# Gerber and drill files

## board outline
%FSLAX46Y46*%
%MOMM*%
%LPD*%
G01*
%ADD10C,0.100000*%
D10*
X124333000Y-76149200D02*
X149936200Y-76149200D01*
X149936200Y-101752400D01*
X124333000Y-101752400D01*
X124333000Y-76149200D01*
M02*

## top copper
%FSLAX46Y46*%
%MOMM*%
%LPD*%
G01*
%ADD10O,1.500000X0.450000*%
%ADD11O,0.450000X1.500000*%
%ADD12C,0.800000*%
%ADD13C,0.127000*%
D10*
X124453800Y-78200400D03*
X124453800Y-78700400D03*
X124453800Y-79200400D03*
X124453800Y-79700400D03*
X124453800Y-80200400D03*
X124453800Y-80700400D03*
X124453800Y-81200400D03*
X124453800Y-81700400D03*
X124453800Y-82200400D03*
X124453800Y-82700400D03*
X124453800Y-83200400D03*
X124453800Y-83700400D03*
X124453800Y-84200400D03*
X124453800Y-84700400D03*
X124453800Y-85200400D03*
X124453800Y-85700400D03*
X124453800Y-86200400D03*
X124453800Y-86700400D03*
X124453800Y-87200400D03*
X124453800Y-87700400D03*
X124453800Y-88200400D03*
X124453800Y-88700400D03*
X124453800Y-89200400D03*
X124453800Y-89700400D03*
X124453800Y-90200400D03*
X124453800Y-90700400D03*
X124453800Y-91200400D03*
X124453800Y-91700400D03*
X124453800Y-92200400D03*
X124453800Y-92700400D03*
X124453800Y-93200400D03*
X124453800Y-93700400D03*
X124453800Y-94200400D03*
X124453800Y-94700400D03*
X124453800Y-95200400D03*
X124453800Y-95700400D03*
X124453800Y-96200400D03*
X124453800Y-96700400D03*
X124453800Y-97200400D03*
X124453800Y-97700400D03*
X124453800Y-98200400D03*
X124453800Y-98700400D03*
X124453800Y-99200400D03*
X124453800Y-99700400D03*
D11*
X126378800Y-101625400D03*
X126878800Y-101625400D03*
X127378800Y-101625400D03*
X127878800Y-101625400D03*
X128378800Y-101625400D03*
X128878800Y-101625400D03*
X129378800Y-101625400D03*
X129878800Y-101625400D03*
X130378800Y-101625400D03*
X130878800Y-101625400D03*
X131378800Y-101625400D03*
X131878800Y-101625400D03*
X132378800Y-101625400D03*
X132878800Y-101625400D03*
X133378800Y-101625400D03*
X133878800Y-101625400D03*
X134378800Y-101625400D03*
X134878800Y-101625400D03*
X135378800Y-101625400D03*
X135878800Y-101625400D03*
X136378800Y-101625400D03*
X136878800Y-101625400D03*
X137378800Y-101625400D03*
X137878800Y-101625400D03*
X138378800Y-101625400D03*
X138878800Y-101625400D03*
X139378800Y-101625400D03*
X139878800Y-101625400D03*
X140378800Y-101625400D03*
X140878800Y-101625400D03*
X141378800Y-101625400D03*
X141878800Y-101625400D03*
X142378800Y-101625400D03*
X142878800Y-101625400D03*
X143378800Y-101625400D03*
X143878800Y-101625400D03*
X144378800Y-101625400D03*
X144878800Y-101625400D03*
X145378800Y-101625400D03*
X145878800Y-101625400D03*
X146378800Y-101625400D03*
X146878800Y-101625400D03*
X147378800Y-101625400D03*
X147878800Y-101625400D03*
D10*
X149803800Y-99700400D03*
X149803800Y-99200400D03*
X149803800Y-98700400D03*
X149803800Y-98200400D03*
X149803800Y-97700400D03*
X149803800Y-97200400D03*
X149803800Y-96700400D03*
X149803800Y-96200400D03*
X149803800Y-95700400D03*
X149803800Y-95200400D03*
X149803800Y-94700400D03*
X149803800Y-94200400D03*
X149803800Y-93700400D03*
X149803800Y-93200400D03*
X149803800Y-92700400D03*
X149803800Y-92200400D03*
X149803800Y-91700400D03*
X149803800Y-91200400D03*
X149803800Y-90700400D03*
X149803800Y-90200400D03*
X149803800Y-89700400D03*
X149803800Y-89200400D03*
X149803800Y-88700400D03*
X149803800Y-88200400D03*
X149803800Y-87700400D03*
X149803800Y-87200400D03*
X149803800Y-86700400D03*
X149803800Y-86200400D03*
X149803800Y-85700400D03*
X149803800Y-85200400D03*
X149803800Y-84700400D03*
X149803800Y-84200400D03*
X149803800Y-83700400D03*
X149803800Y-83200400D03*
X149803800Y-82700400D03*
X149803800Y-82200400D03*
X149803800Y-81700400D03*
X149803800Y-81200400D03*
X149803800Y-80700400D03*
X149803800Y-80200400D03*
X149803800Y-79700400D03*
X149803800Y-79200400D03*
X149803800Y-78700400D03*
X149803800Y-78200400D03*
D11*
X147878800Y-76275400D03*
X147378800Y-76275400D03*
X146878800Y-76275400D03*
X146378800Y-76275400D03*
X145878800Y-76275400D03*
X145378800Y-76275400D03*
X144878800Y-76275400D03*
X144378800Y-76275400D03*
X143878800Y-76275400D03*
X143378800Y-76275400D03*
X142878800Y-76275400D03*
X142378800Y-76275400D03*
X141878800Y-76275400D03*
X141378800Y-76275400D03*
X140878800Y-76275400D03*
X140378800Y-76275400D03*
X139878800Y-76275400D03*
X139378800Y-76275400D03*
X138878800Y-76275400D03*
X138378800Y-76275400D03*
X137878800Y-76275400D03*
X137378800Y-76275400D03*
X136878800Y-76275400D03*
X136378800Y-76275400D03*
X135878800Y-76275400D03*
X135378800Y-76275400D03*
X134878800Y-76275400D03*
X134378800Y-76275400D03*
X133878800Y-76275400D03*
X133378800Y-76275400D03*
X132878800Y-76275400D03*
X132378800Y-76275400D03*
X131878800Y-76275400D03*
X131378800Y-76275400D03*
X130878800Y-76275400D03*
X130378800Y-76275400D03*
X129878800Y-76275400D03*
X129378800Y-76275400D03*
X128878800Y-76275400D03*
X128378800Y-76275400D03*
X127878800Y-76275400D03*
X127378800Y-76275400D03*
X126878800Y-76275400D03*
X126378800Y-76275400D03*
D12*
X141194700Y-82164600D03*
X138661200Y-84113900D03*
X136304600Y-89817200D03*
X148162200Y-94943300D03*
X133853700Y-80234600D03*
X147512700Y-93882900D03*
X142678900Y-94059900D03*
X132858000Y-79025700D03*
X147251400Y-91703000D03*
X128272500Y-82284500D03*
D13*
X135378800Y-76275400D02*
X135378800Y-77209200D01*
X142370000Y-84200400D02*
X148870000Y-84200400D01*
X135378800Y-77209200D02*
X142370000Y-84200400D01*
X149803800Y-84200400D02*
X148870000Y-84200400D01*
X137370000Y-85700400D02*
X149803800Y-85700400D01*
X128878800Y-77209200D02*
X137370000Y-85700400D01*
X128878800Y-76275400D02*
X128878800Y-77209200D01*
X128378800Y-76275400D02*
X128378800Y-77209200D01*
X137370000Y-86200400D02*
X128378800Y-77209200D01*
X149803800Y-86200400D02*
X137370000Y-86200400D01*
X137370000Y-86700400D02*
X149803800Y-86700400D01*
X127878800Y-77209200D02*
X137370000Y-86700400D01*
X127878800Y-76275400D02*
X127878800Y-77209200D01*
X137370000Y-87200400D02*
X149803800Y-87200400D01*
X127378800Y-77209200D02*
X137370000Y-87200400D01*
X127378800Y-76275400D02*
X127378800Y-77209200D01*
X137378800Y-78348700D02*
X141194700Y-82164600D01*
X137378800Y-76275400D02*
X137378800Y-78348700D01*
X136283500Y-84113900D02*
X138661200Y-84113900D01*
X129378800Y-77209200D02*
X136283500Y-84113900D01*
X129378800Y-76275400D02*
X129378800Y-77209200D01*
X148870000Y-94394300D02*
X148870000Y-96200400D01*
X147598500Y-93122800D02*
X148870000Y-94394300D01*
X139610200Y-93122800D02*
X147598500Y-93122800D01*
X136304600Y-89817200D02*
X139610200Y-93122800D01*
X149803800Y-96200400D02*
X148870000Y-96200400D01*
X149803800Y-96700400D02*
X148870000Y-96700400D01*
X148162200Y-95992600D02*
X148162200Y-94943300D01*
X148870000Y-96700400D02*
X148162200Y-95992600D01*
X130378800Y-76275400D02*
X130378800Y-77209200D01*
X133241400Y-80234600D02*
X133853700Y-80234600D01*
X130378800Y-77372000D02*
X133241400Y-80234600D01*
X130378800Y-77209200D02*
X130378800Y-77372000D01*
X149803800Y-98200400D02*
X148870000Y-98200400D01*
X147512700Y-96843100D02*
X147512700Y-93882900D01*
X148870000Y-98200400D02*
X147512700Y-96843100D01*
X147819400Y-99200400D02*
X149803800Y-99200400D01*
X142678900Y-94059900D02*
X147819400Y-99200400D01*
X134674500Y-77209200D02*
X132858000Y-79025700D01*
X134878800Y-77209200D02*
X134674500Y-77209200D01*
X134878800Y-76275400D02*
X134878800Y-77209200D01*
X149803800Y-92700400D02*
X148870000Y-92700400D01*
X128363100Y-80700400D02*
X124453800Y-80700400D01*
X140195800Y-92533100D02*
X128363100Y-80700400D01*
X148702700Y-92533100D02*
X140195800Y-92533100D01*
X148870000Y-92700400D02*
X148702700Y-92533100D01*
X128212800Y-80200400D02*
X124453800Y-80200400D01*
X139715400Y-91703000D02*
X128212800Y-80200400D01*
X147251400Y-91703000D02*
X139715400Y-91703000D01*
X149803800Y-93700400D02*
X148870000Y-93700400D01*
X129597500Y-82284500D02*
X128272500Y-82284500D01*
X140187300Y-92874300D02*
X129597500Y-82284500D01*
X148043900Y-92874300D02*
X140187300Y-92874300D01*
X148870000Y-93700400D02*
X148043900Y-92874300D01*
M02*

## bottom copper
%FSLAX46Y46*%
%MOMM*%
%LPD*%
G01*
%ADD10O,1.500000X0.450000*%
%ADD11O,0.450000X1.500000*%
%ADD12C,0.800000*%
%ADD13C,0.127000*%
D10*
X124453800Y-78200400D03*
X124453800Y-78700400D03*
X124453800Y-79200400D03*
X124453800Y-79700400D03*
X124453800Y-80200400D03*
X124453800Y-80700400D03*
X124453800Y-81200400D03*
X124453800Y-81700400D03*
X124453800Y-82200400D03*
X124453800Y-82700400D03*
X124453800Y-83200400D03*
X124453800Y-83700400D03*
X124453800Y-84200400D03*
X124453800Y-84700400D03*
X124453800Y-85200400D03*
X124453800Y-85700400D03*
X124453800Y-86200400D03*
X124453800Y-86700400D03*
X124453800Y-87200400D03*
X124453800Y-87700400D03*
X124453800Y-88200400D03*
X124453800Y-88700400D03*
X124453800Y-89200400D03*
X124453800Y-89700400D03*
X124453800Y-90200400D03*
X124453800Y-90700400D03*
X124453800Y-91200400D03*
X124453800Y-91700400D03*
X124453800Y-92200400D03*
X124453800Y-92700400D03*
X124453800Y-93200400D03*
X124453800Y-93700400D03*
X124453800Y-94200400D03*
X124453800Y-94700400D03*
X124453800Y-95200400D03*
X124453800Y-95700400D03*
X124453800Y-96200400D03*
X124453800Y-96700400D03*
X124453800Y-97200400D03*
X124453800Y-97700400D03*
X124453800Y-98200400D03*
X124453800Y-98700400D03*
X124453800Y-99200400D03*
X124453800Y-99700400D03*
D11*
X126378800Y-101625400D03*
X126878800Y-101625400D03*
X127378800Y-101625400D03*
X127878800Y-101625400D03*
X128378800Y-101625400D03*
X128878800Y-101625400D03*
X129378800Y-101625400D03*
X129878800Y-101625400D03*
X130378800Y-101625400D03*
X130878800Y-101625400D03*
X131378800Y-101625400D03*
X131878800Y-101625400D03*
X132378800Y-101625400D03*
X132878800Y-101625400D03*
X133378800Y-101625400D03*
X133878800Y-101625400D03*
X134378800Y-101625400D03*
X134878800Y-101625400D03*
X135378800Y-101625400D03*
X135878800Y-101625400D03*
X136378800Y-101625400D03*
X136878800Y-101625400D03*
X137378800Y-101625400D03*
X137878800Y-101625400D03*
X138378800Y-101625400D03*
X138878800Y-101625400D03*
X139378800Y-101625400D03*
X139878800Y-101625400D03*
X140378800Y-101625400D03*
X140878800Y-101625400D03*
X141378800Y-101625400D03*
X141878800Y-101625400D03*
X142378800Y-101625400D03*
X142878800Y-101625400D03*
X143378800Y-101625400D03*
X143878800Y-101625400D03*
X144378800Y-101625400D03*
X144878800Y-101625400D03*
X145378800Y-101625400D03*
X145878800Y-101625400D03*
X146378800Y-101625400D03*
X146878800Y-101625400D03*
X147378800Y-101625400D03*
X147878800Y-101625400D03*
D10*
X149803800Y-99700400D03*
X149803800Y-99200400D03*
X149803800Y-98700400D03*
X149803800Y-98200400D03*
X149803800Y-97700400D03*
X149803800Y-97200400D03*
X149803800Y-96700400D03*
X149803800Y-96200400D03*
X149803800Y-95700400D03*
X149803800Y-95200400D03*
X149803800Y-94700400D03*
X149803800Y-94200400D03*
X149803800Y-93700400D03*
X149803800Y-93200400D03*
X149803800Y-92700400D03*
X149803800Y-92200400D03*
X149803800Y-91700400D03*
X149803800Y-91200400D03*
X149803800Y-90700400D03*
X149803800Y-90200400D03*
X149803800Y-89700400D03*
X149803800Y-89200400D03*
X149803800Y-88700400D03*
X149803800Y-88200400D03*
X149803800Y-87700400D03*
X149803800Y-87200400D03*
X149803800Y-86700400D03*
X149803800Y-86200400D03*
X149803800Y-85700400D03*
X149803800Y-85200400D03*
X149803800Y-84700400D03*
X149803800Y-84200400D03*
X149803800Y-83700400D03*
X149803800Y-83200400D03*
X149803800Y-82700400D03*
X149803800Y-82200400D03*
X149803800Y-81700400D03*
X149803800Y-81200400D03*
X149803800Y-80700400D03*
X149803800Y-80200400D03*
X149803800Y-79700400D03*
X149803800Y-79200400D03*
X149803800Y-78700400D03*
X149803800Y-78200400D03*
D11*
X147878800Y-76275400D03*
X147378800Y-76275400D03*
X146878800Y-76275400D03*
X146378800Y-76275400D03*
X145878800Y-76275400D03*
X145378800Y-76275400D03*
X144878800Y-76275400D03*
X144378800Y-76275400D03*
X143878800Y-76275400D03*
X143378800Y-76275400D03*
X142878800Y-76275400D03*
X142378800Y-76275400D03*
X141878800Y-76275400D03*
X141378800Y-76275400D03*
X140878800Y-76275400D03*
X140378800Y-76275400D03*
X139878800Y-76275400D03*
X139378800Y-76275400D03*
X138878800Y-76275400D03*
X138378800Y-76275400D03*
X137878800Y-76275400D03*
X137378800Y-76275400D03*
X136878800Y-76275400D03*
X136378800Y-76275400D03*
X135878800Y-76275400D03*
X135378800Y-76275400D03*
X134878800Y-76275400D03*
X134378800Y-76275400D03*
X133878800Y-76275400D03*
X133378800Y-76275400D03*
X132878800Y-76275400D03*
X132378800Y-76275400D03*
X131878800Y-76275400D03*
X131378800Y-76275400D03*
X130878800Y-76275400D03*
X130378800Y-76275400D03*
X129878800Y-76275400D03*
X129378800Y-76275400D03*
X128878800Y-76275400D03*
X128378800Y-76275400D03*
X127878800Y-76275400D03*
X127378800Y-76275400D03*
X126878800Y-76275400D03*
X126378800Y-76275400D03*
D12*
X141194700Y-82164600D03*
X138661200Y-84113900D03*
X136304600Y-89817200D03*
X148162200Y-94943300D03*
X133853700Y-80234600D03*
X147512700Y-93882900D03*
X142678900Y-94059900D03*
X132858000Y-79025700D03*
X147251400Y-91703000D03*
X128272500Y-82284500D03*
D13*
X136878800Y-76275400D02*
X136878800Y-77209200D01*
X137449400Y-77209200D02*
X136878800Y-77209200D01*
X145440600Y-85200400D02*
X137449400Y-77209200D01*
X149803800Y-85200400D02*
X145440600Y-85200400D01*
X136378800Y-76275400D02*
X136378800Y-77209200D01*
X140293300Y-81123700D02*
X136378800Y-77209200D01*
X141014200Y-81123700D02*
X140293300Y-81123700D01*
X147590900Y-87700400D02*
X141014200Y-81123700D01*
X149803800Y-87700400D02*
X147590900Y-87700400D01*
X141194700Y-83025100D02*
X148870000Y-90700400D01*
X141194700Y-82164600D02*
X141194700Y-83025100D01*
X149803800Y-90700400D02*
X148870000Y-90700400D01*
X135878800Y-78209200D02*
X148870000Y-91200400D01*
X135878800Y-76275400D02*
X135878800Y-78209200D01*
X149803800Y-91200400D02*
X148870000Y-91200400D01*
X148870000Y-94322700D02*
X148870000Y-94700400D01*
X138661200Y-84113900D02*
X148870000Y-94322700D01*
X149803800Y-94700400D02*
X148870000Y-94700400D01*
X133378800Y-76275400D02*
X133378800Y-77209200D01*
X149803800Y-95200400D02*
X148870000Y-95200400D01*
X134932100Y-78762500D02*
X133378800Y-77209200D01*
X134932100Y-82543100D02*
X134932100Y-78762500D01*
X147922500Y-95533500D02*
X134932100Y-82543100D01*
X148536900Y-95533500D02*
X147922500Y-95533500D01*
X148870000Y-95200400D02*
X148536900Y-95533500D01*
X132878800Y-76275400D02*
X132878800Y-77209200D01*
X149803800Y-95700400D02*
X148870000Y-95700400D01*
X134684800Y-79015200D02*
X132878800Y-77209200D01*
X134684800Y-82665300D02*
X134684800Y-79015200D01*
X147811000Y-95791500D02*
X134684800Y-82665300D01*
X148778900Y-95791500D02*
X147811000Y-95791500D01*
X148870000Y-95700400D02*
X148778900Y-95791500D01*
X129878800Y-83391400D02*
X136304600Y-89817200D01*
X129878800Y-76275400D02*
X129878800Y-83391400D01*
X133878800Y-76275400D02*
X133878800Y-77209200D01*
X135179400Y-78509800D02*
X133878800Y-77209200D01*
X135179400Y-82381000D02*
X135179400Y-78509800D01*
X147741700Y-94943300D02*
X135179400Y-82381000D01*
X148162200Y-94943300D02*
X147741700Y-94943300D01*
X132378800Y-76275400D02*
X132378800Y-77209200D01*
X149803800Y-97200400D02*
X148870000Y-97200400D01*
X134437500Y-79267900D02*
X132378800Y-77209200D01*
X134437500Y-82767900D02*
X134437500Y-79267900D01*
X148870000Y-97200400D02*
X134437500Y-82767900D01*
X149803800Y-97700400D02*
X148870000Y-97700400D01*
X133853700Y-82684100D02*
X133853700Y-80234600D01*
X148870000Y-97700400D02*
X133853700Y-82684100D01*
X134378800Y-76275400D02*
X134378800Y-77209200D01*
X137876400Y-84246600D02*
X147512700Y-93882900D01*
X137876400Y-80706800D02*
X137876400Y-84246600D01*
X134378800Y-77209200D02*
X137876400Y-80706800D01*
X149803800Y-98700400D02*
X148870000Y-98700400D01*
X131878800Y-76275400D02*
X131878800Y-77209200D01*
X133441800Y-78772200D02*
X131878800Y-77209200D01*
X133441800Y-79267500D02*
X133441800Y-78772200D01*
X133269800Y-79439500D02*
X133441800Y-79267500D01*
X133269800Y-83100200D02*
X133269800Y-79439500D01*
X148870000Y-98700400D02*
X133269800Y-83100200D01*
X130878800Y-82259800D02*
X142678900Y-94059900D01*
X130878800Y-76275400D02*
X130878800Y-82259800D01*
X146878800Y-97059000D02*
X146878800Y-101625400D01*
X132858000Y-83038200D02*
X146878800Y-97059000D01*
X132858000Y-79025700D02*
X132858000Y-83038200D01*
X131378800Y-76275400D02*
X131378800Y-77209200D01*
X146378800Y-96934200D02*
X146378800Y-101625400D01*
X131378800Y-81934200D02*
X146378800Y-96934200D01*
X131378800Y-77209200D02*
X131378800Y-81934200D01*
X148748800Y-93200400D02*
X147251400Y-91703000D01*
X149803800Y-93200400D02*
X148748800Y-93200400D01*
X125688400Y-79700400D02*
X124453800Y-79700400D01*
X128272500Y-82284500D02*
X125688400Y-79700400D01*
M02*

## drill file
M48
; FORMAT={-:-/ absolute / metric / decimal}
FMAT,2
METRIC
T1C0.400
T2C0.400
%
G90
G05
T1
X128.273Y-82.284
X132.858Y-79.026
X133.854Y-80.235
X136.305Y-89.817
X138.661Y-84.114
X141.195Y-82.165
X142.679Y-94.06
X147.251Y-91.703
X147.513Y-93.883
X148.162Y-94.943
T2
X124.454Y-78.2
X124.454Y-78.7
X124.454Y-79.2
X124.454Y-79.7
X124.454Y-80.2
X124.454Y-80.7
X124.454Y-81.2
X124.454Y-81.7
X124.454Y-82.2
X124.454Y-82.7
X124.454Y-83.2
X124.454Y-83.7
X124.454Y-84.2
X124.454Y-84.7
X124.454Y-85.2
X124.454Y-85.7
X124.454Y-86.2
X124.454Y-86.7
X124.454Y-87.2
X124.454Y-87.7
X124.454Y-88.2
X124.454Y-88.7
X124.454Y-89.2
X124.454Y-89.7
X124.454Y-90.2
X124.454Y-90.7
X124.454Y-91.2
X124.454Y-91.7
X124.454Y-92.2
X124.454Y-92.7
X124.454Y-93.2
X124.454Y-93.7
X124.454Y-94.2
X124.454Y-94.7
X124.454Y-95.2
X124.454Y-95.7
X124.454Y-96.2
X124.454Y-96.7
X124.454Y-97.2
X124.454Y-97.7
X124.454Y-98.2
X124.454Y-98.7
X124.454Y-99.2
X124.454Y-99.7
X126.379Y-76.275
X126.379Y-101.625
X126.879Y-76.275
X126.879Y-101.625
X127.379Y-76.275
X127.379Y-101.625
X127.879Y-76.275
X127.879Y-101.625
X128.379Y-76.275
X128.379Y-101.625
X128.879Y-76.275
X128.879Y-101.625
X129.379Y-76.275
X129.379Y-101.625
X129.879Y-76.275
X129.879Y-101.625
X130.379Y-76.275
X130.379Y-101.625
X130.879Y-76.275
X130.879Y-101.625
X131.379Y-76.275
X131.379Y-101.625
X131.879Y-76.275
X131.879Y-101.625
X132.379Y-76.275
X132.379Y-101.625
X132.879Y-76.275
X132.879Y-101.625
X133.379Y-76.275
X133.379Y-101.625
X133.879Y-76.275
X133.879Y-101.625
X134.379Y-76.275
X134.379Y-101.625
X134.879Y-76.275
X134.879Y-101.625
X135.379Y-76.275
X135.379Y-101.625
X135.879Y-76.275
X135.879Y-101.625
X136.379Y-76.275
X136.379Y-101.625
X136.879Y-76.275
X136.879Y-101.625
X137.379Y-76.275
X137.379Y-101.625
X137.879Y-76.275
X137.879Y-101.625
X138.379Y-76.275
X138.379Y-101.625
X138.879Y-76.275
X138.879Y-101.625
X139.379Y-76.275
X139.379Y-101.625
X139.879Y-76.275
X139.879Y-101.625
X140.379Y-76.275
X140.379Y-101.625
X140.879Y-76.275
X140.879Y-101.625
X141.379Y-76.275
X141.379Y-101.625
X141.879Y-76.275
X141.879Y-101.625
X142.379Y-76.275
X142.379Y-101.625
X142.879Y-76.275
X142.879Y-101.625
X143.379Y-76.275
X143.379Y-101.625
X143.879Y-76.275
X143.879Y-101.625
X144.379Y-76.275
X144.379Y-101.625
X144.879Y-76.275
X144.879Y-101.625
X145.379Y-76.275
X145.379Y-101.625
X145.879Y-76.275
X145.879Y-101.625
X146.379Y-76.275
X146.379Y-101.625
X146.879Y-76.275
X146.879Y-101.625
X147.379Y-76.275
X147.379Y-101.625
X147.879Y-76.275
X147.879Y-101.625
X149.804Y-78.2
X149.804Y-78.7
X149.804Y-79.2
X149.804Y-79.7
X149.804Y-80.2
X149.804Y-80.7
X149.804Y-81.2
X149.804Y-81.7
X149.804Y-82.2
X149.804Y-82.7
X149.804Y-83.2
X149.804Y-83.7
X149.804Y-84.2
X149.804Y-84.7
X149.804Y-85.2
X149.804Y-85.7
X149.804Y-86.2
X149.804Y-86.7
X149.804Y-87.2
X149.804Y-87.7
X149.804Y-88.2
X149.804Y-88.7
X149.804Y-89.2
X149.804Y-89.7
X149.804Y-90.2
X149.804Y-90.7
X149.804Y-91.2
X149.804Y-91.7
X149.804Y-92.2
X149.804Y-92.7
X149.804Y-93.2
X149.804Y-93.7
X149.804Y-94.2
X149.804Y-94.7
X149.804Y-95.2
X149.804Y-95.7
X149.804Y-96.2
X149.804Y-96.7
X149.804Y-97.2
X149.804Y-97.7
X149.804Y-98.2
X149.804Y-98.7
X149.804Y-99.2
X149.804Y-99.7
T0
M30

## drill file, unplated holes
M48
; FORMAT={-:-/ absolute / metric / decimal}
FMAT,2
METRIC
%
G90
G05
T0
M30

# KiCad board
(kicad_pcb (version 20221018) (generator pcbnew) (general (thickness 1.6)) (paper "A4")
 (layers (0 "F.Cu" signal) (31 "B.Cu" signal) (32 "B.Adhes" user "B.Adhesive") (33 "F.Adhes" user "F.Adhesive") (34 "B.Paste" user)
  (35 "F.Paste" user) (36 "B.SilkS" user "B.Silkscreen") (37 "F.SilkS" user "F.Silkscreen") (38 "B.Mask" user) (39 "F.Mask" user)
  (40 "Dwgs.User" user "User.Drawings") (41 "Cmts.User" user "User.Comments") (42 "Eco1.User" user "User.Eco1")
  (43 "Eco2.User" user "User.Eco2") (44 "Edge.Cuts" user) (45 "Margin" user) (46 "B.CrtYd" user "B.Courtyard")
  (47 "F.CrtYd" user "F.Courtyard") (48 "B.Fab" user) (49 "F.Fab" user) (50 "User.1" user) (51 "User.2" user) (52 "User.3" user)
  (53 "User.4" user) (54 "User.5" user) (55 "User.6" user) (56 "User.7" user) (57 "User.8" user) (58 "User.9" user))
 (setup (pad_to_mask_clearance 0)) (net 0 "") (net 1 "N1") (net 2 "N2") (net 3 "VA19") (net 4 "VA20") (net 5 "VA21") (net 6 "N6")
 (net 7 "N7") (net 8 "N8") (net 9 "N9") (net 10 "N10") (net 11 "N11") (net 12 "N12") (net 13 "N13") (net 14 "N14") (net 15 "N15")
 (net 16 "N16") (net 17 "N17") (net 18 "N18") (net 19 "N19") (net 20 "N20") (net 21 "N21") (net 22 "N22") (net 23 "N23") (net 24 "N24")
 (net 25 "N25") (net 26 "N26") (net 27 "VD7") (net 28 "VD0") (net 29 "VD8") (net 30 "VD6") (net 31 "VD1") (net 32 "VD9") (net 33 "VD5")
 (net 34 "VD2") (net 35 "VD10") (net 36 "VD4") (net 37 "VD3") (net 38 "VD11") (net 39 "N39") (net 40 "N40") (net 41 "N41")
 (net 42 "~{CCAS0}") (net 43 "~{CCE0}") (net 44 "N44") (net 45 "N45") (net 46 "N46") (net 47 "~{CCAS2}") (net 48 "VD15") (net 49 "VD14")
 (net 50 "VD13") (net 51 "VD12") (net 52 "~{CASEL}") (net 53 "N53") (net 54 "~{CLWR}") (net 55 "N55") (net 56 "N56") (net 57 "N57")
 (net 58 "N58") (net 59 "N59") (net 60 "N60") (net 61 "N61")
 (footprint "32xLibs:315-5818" (layer "F.Cu") (at 137.1288 88.9504)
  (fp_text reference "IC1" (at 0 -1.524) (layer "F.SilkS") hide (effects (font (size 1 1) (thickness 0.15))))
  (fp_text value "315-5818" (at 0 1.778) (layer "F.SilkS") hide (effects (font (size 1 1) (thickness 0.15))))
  (pad "1" thru_hole oval (at -12.675 -10.75) (size 1.5 0.45) (drill 0.4) (layers "*.Cu" "*.Mask"))
  (pad "2" thru_hole oval (at -12.675 -10.25) (size 1.5 0.45) (drill 0.4) (layers "*.Cu" "*.Mask") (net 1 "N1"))
  (pad "3" thru_hole oval (at -12.675 -9.75) (size 1.5 0.45) (drill 0.4) (layers "*.Cu" "*.Mask") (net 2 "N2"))
  (pad "4" thru_hole oval (at -12.675 -9.25) (size 1.5 0.45) (drill 0.4) (layers "*.Cu" "*.Mask") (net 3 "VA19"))
  (pad "5" thru_hole oval (at -12.675 -8.75) (size 1.5 0.45) (drill 0.4) (layers "*.Cu" "*.Mask") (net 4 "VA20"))
  (pad "6" thru_hole oval (at -12.675 -8.25) (size 1.5 0.45) (drill 0.4) (layers "*.Cu" "*.Mask") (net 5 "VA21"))
  (pad "7" thru_hole oval (at -12.675 -7.75) (size 1.5 0.45) (drill 0.4) (layers "*.Cu" "*.Mask") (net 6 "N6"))
  (pad "8" thru_hole oval (at -12.675 -7.25) (size 1.5 0.45) (drill 0.4) (layers "*.Cu" "*.Mask") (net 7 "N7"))
  (pad "9" thru_hole oval (at -12.675 -6.75) (size 1.5 0.45) (drill 0.4) (layers "*.Cu" "*.Mask"))
  (pad "10" thru_hole oval (at -12.675 -6.25) (size 1.5 0.45) (drill 0.4) (layers "*.Cu" "*.Mask"))
  (pad "11" thru_hole oval (at -12.675 -5.75) (size 1.5 0.45) (drill 0.4) (layers "*.Cu" "*.Mask"))
  (pad "12" thru_hole oval (at -12.675 -5.25) (size 1.5 0.45) (drill 0.4) (layers "*.Cu" "*.Mask"))
  (pad "13" thru_hole oval (at -12.675 -4.75) (size 1.5 0.45) (drill 0.4) (layers "*.Cu" "*.Mask"))
  (pad "14" thru_hole oval (at -12.675 -4.25) (size 1.5 0.45) (drill 0.4) (layers "*.Cu" "*.Mask"))
  (pad "15" thru_hole oval (at -12.675 -3.75) (size 1.5 0.45) (drill 0.4) (layers "*.Cu" "*.Mask"))
  (pad "16" thru_hole oval (at -12.675 -3.25) (size 1.5 0.45) (drill 0.4) (layers "*.Cu" "*.Mask"))
  (pad "17" thru_hole oval (at -12.675 -2.75) (size 1.5 0.45) (drill 0.4) (layers "*.Cu" "*.Mask"))
  (pad "18" thru_hole oval (at -12.675 -2.25) (size 1.5 0.45) (drill 0.4) (layers "*.Cu" "*.Mask"))
  (pad "19" thru_hole oval (at -12.675 -1.75) (size 1.5 0.45) (drill 0.4) (layers "*.Cu" "*.Mask"))
  (pad "20" thru_hole oval (at -12.675 -1.25) (size 1.5 0.45) (drill 0.4) (layers "*.Cu" "*.Mask"))
  (pad "21" thru_hole oval (at -12.675 -0.75) (size 1.5 0.45) (drill 0.4) (layers "*.Cu" "*.Mask"))
  (pad "22" thru_hole oval (at -12.675 -0.25) (size 1.5 0.45) (drill 0.4) (layers "*.Cu" "*.Mask"))
  (pad "23" thru_hole oval (at -12.675 0.25) (size 1.5 0.45) (drill 0.4) (layers "*.Cu" "*.Mask"))
  (pad "24" thru_hole oval (at -12.675 0.75) (size 1.5 0.45) (drill 0.4) (layers "*.Cu" "*.Mask"))
  (pad "25" thru_hole oval (at -12.675 1.25) (size 1.5 0.45) (drill 0.4) (layers "*.Cu" "*.Mask"))
  (pad "26" thru_hole oval (at -12.675 1.75) (size 1.5 0.45) (drill 0.4) (layers "*.Cu" "*.Mask"))
  (pad "27" thru_hole oval (at -12.675 2.25) (size 1.5 0.45) (drill 0.4) (layers "*.Cu" "*.Mask"))
  (pad "28" thru_hole oval (at -12.675 2.75) (size 1.5 0.45) (drill 0.4) (layers "*.Cu" "*.Mask"))
  (pad "29" thru_hole oval (at -12.675 3.25) (size 1.5 0.45) (drill 0.4) (layers "*.Cu" "*.Mask"))
  (pad "30" thru_hole oval (at -12.675 3.75) (size 1.5 0.45) (drill 0.4) (layers "*.Cu" "*.Mask"))
  (pad "31" thru_hole oval (at -12.675 4.25) (size 1.5 0.45) (drill 0.4) (layers "*.Cu" "*.Mask"))
  (pad "32" thru_hole oval (at -12.675 4.75) (size 1.5 0.45) (drill 0.4) (layers "*.Cu" "*.Mask"))
  (pad "33" thru_hole oval (at -12.675 5.25) (size 1.5 0.45) (drill 0.4) (layers "*.Cu" "*.Mask") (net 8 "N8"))
  (pad "34" thru_hole oval (at -12.675 5.75) (size 1.5 0.45) (drill 0.4) (layers "*.Cu" "*.Mask"))
  (pad "35" thru_hole oval (at -12.675 6.25) (size 1.5 0.45) (drill 0.4) (layers "*.Cu" "*.Mask"))
  (pad "36" thru_hole oval (at -12.675 6.75) (size 1.5 0.45) (drill 0.4) (layers "*.Cu" "*.Mask"))
  (pad "37" thru_hole oval (at -12.675 7.25) (size 1.5 0.45) (drill 0.4) (layers "*.Cu" "*.Mask"))
  (pad "38" thru_hole oval (at -12.675 7.75) (size 1.5 0.45) (drill 0.4) (layers "*.Cu" "*.Mask"))
  (pad "39" thru_hole oval (at -12.675 8.25) (size 1.5 0.45) (drill 0.4) (layers "*.Cu" "*.Mask"))
  (pad "40" thru_hole oval (at -12.675 8.75) (size 1.5 0.45) (drill 0.4) (layers "*.Cu" "*.Mask"))
  (pad "41" thru_hole oval (at -12.675 9.25) (size 1.5 0.45) (drill 0.4) (layers "*.Cu" "*.Mask"))
  (pad "42" thru_hole oval (at -12.675 9.75) (size 1.5 0.45) (drill 0.4) (layers "*.Cu" "*.Mask"))
  (pad "43" thru_hole oval (at -12.675 10.25) (size 1.5 0.45) (drill 0.4) (layers "*.Cu" "*.Mask"))
  (pad "44" thru_hole oval (at -12.675 10.75) (size 1.5 0.45) (drill 0.4) (layers "*.Cu" "*.Mask"))
  (pad "45" thru_hole oval (at -10.75 12.675) (size 0.45 1.5) (drill 0.4) (layers "*.Cu" "*.Mask"))
  (pad "46" thru_hole oval (at -10.25 12.675) (size 0.45 1.5) (drill 0.4) (layers "*.Cu" "*.Mask"))
  (pad "47" thru_hole oval (at -9.75 12.675) (size 0.45 1.5) (drill 0.4) (layers "*.Cu" "*.Mask"))
  (pad "48" thru_hole oval (at -9.25 12.675) (size 0.45 1.5) (drill 0.4) (layers "*.Cu" "*.Mask"))
  (pad "49" thru_hole oval (at -8.75 12.675) (size 0.45 1.5) (drill 0.4) (layers "*.Cu" "*.Mask"))
  (pad "50" thru_hole oval (at -8.25 12.675) (size 0.45 1.5) (drill 0.4) (layers "*.Cu" "*.Mask"))
  (pad "51" thru_hole oval (at -7.75 12.675) (size 0.45 1.5) (drill 0.4) (layers "*.Cu" "*.Mask"))
  (pad "52" thru_hole oval (at -7.25 12.675) (size 0.45 1.5) (drill 0.4) (layers "*.Cu" "*.Mask"))
  (pad "53" thru_hole oval (at -6.75 12.675) (size 0.45 1.5) (drill 0.4) (layers "*.Cu" "*.Mask"))
  (pad "54" thru_hole oval (at -6.25 12.675) (size 0.45 1.5) (drill 0.4) (layers "*.Cu" "*.Mask"))
  (pad "55" thru_hole oval (at -5.75 12.675) (size 0.45 1.5) (drill 0.4) (layers "*.Cu" "*.Mask"))
  (pad "56" thru_hole oval (at -5.25 12.675) (size 0.45 1.5) (drill 0.4) (layers "*.Cu" "*.Mask"))
  (pad "57" thru_hole oval (at -4.75 12.675) (size 0.45 1.5) (drill 0.4) (layers "*.Cu" "*.Mask"))
  (pad "58" thru_hole oval (at -4.25 12.675) (size 0.45 1.5) (drill 0.4) (layers "*.Cu" "*.Mask"))
  (pad "59" thru_hole oval (at -3.75 12.675) (size 0.45 1.5) (drill 0.4) (layers "*.Cu" "*.Mask"))
  (pad "60" thru_hole oval (at -3.25 12.675) (size 0.45 1.5) (drill 0.4) (layers "*.Cu" "*.Mask"))
  (pad "61" thru_hole oval (at -2.75 12.675) (size 0.45 1.5) (drill 0.4) (layers "*.Cu" "*.Mask"))
  (pad "62" thru_hole oval (at -2.25 12.675) (size 0.45 1.5) (drill 0.4) (layers "*.Cu" "*.Mask"))
  (pad "63" thru_hole oval (at -1.75 12.675) (size 0.45 1.5) (drill 0.4) (layers "*.Cu" "*.Mask"))
  (pad "64" thru_hole oval (at -1.25 12.675) (size 0.45 1.5) (drill 0.4) (layers "*.Cu" "*.Mask"))
  (pad "65" thru_hole oval (at -0.75 12.675) (size 0.45 1.5) (drill 0.4) (layers "*.Cu" "*.Mask"))
  (pad "66" thru_hole oval (at -0.25 12.675) (size 0.45 1.5) (drill 0.4) (layers "*.Cu" "*.Mask"))
  (pad "67" thru_hole oval (at 0.25 12.675) (size 0.45 1.5) (drill 0.4) (layers "*.Cu" "*.Mask") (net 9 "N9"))
  (pad "68" thru_hole oval (at 0.75 12.675) (size 0.45 1.5) (drill 0.4) (layers "*.Cu" "*.Mask") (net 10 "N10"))
  (pad "69" thru_hole oval (at 1.25 12.675) (size 0.45 1.5) (drill 0.4) (layers "*.Cu" "*.Mask") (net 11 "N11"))
  (pad "70" thru_hole oval (at 1.75 12.675) (size 0.45 1.5) (drill 0.4) (layers "*.Cu" "*.Mask") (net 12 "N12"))
  (pad "71" thru_hole oval (at 2.25 12.675) (size 0.45 1.5) (drill 0.4) (layers "*.Cu" "*.Mask") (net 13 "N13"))
  (pad "72" thru_hole oval (at 2.75 12.675) (size 0.45 1.5) (drill 0.4) (layers "*.Cu" "*.Mask") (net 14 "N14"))
  (pad "73" thru_hole oval (at 3.25 12.675) (size 0.45 1.5) (drill 0.4) (layers "*.Cu" "*.Mask") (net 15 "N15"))
  (pad "74" thru_hole oval (at 3.75 12.675) (size 0.45 1.5) (drill 0.4) (layers "*.Cu" "*.Mask") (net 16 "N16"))
  (pad "75" thru_hole oval (at 4.25 12.675) (size 0.45 1.5) (drill 0.4) (layers "*.Cu" "*.Mask") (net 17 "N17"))
  (pad "76" thru_hole oval (at 4.75 12.675) (size 0.45 1.5) (drill 0.4) (layers "*.Cu" "*.Mask") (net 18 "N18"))
  (pad "77" thru_hole oval (at 5.25 12.675) (size 0.45 1.5) (drill 0.4) (layers "*.Cu" "*.Mask") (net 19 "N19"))
  (pad "78" thru_hole oval (at 5.75 12.675) (size 0.45 1.5) (drill 0.4) (layers "*.Cu" "*.Mask") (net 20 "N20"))
  (pad "79" thru_hole oval (at 6.25 12.675) (size 0.45 1.5) (drill 0.4) (layers "*.Cu" "*.Mask") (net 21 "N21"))
  (pad "80" thru_hole oval (at 6.75 12.675) (size 0.45 1.5) (drill 0.4) (layers "*.Cu" "*.Mask") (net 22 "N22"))
  (pad "81" thru_hole oval (at 7.25 12.675) (size 0.45 1.5) (drill 0.4) (layers "*.Cu" "*.Mask") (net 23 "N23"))
  (pad "82" thru_hole oval (at 7.75 12.675) (size 0.45 1.5) (drill 0.4) (layers "*.Cu" "*.Mask") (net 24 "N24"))
  (pad "83" thru_hole oval (at 8.25 12.675) (size 0.45 1.5) (drill 0.4) (layers "*.Cu" "*.Mask") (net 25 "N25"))
  (pad "84" thru_hole oval (at 8.75 12.675) (size 0.45 1.5) (drill 0.4) (layers "*.Cu" "*.Mask") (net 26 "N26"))
  (pad "85" thru_hole oval (at 9.25 12.675) (size 0.45 1.5) (drill 0.4) (layers "*.Cu" "*.Mask") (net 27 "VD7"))
  (pad "86" thru_hole oval (at 9.75 12.675) (size 0.45 1.5) (drill 0.4) (layers "*.Cu" "*.Mask") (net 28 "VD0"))
  (pad "87" thru_hole oval (at 10.25 12.675) (size 0.45 1.5) (drill 0.4) (layers "*.Cu" "*.Mask"))
  (pad "88" thru_hole oval (at 10.75 12.675) (size 0.45 1.5) (drill 0.4) (layers "*.Cu" "*.Mask"))
  (pad "89" thru_hole oval (at 12.675 10.75) (size 1.5 0.45) (drill 0.4) (layers "*.Cu" "*.Mask"))
  (pad "90" thru_hole oval (at 12.675 10.25) (size 1.5 0.45) (drill 0.4) (layers "*.Cu" "*.Mask") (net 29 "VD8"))
  (pad "91" thru_hole oval (at 12.675 9.75) (size 1.5 0.45) (drill 0.4) (layers "*.Cu" "*.Mask") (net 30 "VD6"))
  (pad "92" thru_hole oval (at 12.675 9.25) (size 1.5 0.45) (drill 0.4) (layers "*.Cu" "*.Mask") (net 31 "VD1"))
  (pad "93" thru_hole oval (at 12.675 8.75) (size 1.5 0.45) (drill 0.4) (layers "*.Cu" "*.Mask") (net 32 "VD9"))
  (pad "94" thru_hole oval (at 12.675 8.25) (size 1.5 0.45) (drill 0.4) (layers "*.Cu" "*.Mask") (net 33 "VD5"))
  (pad "95" thru_hole oval (at 12.675 7.75) (size 1.5 0.45) (drill 0.4) (layers "*.Cu" "*.Mask") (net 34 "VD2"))
  (pad "96" thru_hole oval (at 12.675 7.25) (size 1.5 0.45) (drill 0.4) (layers "*.Cu" "*.Mask") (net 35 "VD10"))
  (pad "97" thru_hole oval (at 12.675 6.75) (size 1.5 0.45) (drill 0.4) (layers "*.Cu" "*.Mask") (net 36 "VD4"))
  (pad "98" thru_hole oval (at 12.675 6.25) (size 1.5 0.45) (drill 0.4) (layers "*.Cu" "*.Mask") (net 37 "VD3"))
  (pad "99" thru_hole oval (at 12.675 5.75) (size 1.5 0.45) (drill 0.4) (layers "*.Cu" "*.Mask") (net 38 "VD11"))
  (pad "100" thru_hole oval (at 12.675 5.25) (size 1.5 0.45) (drill 0.4) (layers "*.Cu" "*.Mask") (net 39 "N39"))
  (pad "101" thru_hole oval (at 12.675 4.75) (size 1.5 0.45) (drill 0.4) (layers "*.Cu" "*.Mask") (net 3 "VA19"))
  (pad "102" thru_hole oval (at 12.675 4.25) (size 1.5 0.45) (drill 0.4) (layers "*.Cu" "*.Mask") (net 4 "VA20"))
  (pad "103" thru_hole oval (at 12.675 3.75) (size 1.5 0.45) (drill 0.4) (layers "*.Cu" "*.Mask") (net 5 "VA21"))
  (pad "104" thru_hole oval (at 12.675 3.25) (size 1.5 0.45) (drill 0.4) (layers "*.Cu" "*.Mask") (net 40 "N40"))
  (pad "105" thru_hole oval (at 12.675 2.75) (size 1.5 0.45) (drill 0.4) (layers "*.Cu" "*.Mask") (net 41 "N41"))
  (pad "106" thru_hole oval (at 12.675 2.25) (size 1.5 0.45) (drill 0.4) (layers "*.Cu" "*.Mask") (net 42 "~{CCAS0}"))
  (pad "107" thru_hole oval (at 12.675 1.75) (size 1.5 0.45) (drill 0.4) (layers "*.Cu" "*.Mask") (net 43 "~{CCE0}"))
  (pad "108" thru_hole oval (at 12.675 1.25) (size 1.5 0.45) (drill 0.4) (layers "*.Cu" "*.Mask") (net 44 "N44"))
  (pad "109" thru_hole oval (at 12.675 0.75) (size 1.5 0.45) (drill 0.4) (layers "*.Cu" "*.Mask") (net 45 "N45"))
  (pad "110" thru_hole oval (at 12.675 0.25) (size 1.5 0.45) (drill 0.4) (layers "*.Cu" "*.Mask"))
  (pad "111" thru_hole oval (at 12.675 -0.25) (size 1.5 0.45) (drill 0.4) (layers "*.Cu" "*.Mask"))
  (pad "112" thru_hole oval (at 12.675 -0.75) (size 1.5 0.45) (drill 0.4) (layers "*.Cu" "*.Mask") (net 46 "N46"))
  (pad "113" thru_hole oval (at 12.675 -1.25) (size 1.5 0.45) (drill 0.4) (layers "*.Cu" "*.Mask") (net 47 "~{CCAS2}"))
  (pad "114" thru_hole oval (at 12.675 -1.75) (size 1.5 0.45) (drill 0.4) (layers "*.Cu" "*.Mask") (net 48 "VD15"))
  (pad "115" thru_hole oval (at 12.675 -2.25) (size 1.5 0.45) (drill 0.4) (layers "*.Cu" "*.Mask") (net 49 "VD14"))
  (pad "116" thru_hole oval (at 12.675 -2.75) (size 1.5 0.45) (drill 0.4) (layers "*.Cu" "*.Mask") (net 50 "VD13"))
  (pad "117" thru_hole oval (at 12.675 -3.25) (size 1.5 0.45) (drill 0.4) (layers "*.Cu" "*.Mask") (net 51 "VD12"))
  (pad "118" thru_hole oval (at 12.675 -3.75) (size 1.5 0.45) (drill 0.4) (layers "*.Cu" "*.Mask") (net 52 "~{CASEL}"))
  (pad "119" thru_hole oval (at 12.675 -4.25) (size 1.5 0.45) (drill 0.4) (layers "*.Cu" "*.Mask") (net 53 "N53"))
  (pad "120" thru_hole oval (at 12.675 -4.75) (size 1.5 0.45) (drill 0.4) (layers "*.Cu" "*.Mask") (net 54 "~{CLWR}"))
  (pad "121" thru_hole oval (at 12.675 -5.25) (size 1.5 0.45) (drill 0.4) (layers "*.Cu" "*.Mask") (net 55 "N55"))
  (pad "122" thru_hole oval (at 12.675 -5.75) (size 1.5 0.45) (drill 0.4) (layers "*.Cu" "*.Mask"))
  (pad "123" thru_hole oval (at 12.675 -6.25) (size 1.5 0.45) (drill 0.4) (layers "*.Cu" "*.Mask"))
  (pad "124" thru_hole oval (at 12.675 -6.75) (size 1.5 0.45) (drill 0.4) (layers "*.Cu" "*.Mask"))
  (pad "125" thru_hole oval (at 12.675 -7.25) (size 1.5 0.45) (drill 0.4) (layers "*.Cu" "*.Mask"))
  (pad "126" thru_hole oval (at 12.675 -7.75) (size 1.5 0.45) (drill 0.4) (layers "*.Cu" "*.Mask"))
  (pad "127" thru_hole oval (at 12.675 -8.25) (size 1.5 0.45) (drill 0.4) (layers "*.Cu" "*.Mask"))
  (pad "128" thru_hole oval (at 12.675 -8.75) (size 1.5 0.45) (drill 0.4) (layers "*.Cu" "*.Mask") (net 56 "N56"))
  (pad "129" thru_hole oval (at 12.675 -9.25) (size 1.5 0.45) (drill 0.4) (layers "*.Cu" "*.Mask") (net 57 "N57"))
  (pad "130" thru_hole oval (at 12.675 -9.75) (size 1.5 0.45) (drill 0.4) (layers "*.Cu" "*.Mask") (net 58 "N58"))
  (pad "131" thru_hole oval (at 12.675 -10.25) (size 1.5 0.45) (drill 0.4) (layers "*.Cu" "*.Mask"))
  (pad "132" thru_hole oval (at 12.675 -10.75) (size 1.5 0.45) (drill 0.4) (layers "*.Cu" "*.Mask"))
  (pad "133" thru_hole oval (at 10.75 -12.675) (size 0.45 1.5) (drill 0.4) (layers "*.Cu" "*.Mask"))
  (pad "134" thru_hole oval (at 10.25 -12.675) (size 0.45 1.5) (drill 0.4) (layers "*.Cu" "*.Mask"))
  (pad "135" thru_hole oval (at 9.75 -12.675) (size 0.45 1.5) (drill 0.4) (layers "*.Cu" "*.Mask"))
  (pad "136" thru_hole oval (at 9.25 -12.675) (size 0.45 1.5) (drill 0.4) (layers "*.Cu" "*.Mask"))
  (pad "137" thru_hole oval (at 8.75 -12.675) (size 0.45 1.5) (drill 0.4) (layers "*.Cu" "*.Mask"))
  (pad "138" thru_hole oval (at 8.25 -12.675) (size 0.45 1.5) (drill 0.4) (layers "*.Cu" "*.Mask"))
  (pad "139" thru_hole oval (at 7.75 -12.675) (size 0.45 1.5) (drill 0.4) (layers "*.Cu" "*.Mask"))
  (pad "140" thru_hole oval (at 7.25 -12.675) (size 0.45 1.5) (drill 0.4) (layers "*.Cu" "*.Mask"))
  (pad "141" thru_hole oval (at 6.75 -12.675) (size 0.45 1.5) (drill 0.4) (layers "*.Cu" "*.Mask"))
  (pad "142" thru_hole oval (at 6.25 -12.675) (size 0.45 1.5) (drill 0.4) (layers "*.Cu" "*.Mask"))
  (pad "143" thru_hole oval (at 5.75 -12.675) (size 0.45 1.5) (drill 0.4) (layers "*.Cu" "*.Mask"))
  (pad "144" thru_hole oval (at 5.25 -12.675) (size 0.45 1.5) (drill 0.4) (layers "*.Cu" "*.Mask"))
  (pad "145" thru_hole oval (at 4.75 -12.675) (size 0.45 1.5) (drill 0.4) (layers "*.Cu" "*.Mask"))
  (pad "146" thru_hole oval (at 4.25 -12.675) (size 0.45 1.5) (drill 0.4) (layers "*.Cu" "*.Mask"))
  (pad "147" thru_hole oval (at 3.75 -12.675) (size 0.45 1.5) (drill 0.4) (layers "*.Cu" "*.Mask"))
  (pad "148" thru_hole oval (at 3.25 -12.675) (size 0.45 1.5) (drill 0.4) (layers "*.Cu" "*.Mask"))
  (pad "149" thru_hole oval (at 2.75 -12.675) (size 0.45 1.5) (drill 0.4) (layers "*.Cu" "*.Mask"))
  (pad "150" thru_hole oval (at 2.25 -12.675) (size 0.45 1.5) (drill 0.4) (layers "*.Cu" "*.Mask"))
  (pad "151" thru_hole oval (at 1.75 -12.675) (size 0.45 1.5) (drill 0.4) (layers "*.Cu" "*.Mask") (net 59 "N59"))
  (pad "152" thru_hole oval (at 1.25 -12.675) (size 0.45 1.5) (drill 0.4) (layers "*.Cu" "*.Mask") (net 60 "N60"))
  (pad "153" thru_hole oval (at 0.75 -12.675) (size 0.45 1.5) (drill 0.4) (layers "*.Cu" "*.Mask") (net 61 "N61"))
  (pad "154" thru_hole oval (at 0.25 -12.675) (size 0.45 1.5) (drill 0.4) (layers "*.Cu" "*.Mask") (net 43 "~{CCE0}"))
  (pad "155" thru_hole oval (at -0.25 -12.675) (size 0.45 1.5) (drill 0.4) (layers "*.Cu" "*.Mask") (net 52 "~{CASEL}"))
  (pad "156" thru_hole oval (at -0.75 -12.675) (size 0.45 1.5) (drill 0.4) (layers "*.Cu" "*.Mask") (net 47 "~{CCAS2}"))
  (pad "157" thru_hole oval (at -1.25 -12.675) (size 0.45 1.5) (drill 0.4) (layers "*.Cu" "*.Mask") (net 42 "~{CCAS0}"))
  (pad "158" thru_hole oval (at -1.75 -12.675) (size 0.45 1.5) (drill 0.4) (layers "*.Cu" "*.Mask") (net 54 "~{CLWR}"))
  (pad "159" thru_hole oval (at -2.25 -12.675) (size 0.45 1.5) (drill 0.4) (layers "*.Cu" "*.Mask") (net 28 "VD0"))
  (pad "160" thru_hole oval (at -2.75 -12.675) (size 0.45 1.5) (drill 0.4) (layers "*.Cu" "*.Mask") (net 31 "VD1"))
  (pad "161" thru_hole oval (at -3.25 -12.675) (size 0.45 1.5) (drill 0.4) (layers "*.Cu" "*.Mask") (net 34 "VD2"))
  (pad "162" thru_hole oval (at -3.75 -12.675) (size 0.45 1.5) (drill 0.4) (layers "*.Cu" "*.Mask") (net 37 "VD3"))
  (pad "163" thru_hole oval (at -4.25 -12.675) (size 0.45 1.5) (drill 0.4) (layers "*.Cu" "*.Mask") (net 36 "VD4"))
  (pad "164" thru_hole oval (at -4.75 -12.675) (size 0.45 1.5) (drill 0.4) (layers "*.Cu" "*.Mask") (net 33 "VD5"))
  (pad "165" thru_hole oval (at -5.25 -12.675) (size 0.45 1.5) (drill 0.4) (layers "*.Cu" "*.Mask") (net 30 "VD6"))
  (pad "166" thru_hole oval (at -5.75 -12.675) (size 0.45 1.5) (drill 0.4) (layers "*.Cu" "*.Mask") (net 27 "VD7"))
  (pad "167" thru_hole oval (at -6.25 -12.675) (size 0.45 1.5) (drill 0.4) (layers "*.Cu" "*.Mask") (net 29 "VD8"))
  (pad "168" thru_hole oval (at -6.75 -12.675) (size 0.45 1.5) (drill 0.4) (layers "*.Cu" "*.Mask") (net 32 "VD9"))
  (pad "169" thru_hole oval (at -7.25 -12.675) (size 0.45 1.5) (drill 0.4) (layers "*.Cu" "*.Mask") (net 35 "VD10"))
  (pad "170" thru_hole oval (at -7.75 -12.675) (size 0.45 1.5) (drill 0.4) (layers "*.Cu" "*.Mask") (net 38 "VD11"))
  (pad "171" thru_hole oval (at -8.25 -12.675) (size 0.45 1.5) (drill 0.4) (layers "*.Cu" "*.Mask") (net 51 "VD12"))
  (pad "172" thru_hole oval (at -8.75 -12.675) (size 0.45 1.5) (drill 0.4) (layers "*.Cu" "*.Mask") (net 50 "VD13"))
  (pad "173" thru_hole oval (at -9.25 -12.675) (size 0.45 1.5) (drill 0.4) (layers "*.Cu" "*.Mask") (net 49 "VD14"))
  (pad "174" thru_hole oval (at -9.75 -12.675) (size 0.45 1.5) (drill 0.4) (layers "*.Cu" "*.Mask") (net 48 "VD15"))
  (pad "175" thru_hole oval (at -10.25 -12.675) (size 0.45 1.5) (drill 0.4) (layers "*.Cu" "*.Mask"))
  (pad "176" thru_hole oval (at -10.75 -12.675) (size 0.45 1.5) (drill 0.4) (layers "*.Cu" "*.Mask")))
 (gr_rect (start 124.333 76.1492) (end 149.9362 101.7524) (stroke (width 0.1) (type default)) (fill none) (layer "Edge.Cuts"))
 (segment (start 148.0439 92.8743) (end 140.1873 92.8743) (width 0.127) (layer "F.Cu") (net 3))
 (segment (start 149.8038 93.7004) (end 148.87 93.7004) (width 0.127) (layer "F.Cu") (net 3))
 (segment (start 129.5975 82.2845) (end 128.2725 82.2845) (width 0.127) (layer "F.Cu") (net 3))
 (segment (start 140.1873 92.8743) (end 129.5975 82.2845) (width 0.127) (layer "F.Cu") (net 3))
 (segment (start 148.87 93.7004) (end 148.0439 92.8743) (width 0.127) (layer "F.Cu") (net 3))
 (via (at 128.2725 82.2845) (size 0.8) (drill 0.4) (layers "F.Cu" "B.Cu") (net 3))
 (segment (start 125.6884 79.7004) (end 124.4538 79.7004) (width 0.127) (layer "B.Cu") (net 3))
 (segment (start 128.2725 82.2845) (end 125.6884 79.7004) (width 0.127) (layer "B.Cu") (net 3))
 (segment (start 147.2514 91.703) (end 139.7154 91.703) (width 0.127) (layer "F.Cu") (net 4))
 (segment (start 139.7154 91.703) (end 128.2128 80.2004) (width 0.127) (layer "F.Cu") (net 4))
 (segment (start 128.2128 80.2004) (end 124.4538 80.2004) (width 0.127) (layer "F.Cu") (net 4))
 (via (at 147.2514 91.703) (size 0.8) (drill 0.4) (layers "F.Cu" "B.Cu") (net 4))
 (segment (start 149.8038 93.2004) (end 148.7488 93.2004) (width 0.127) (layer "B.Cu") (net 4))
 (segment (start 148.7488 93.2004) (end 147.2514 91.703) (width 0.127) (layer "B.Cu") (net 4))
 (segment (start 149.8038 92.7004) (end 148.87 92.7004) (width 0.127) (layer "F.Cu") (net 5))
 (segment (start 148.7027 92.5331) (end 140.1958 92.5331) (width 0.127) (layer "F.Cu") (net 5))
 (segment (start 128.3631 80.7004) (end 124.4538 80.7004) (width 0.127) (layer "F.Cu") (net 5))
 (segment (start 140.1958 92.5331) (end 128.3631 80.7004) (width 0.127) (layer "F.Cu") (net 5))
 (segment (start 148.87 92.7004) (end 148.7027 92.5331) (width 0.127) (layer "F.Cu") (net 5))
 (segment (start 131.3788 81.9342) (end 146.3788 96.9342) (width 0.127) (layer "B.Cu") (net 27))
 (segment (start 131.3788 76.2754) (end 131.3788 77.2092) (width 0.127) (layer "B.Cu") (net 27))
 (segment (start 131.3788 77.2092) (end 131.3788 81.9342) (width 0.127) (layer "B.Cu") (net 27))
 (segment (start 146.3788 96.9342) (end 146.3788 101.6254) (width 0.127) (layer "B.Cu") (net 27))
 (segment (start 134.6745 77.2092) (end 132.858 79.0257) (width 0.127) (layer "F.Cu") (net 28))
 (segment (start 134.8788 76.2754) (end 134.8788 77.2092) (width 0.127) (layer "F.Cu") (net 28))
 (segment (start 134.8788 77.2092) (end 134.6745 77.2092) (width 0.127) (layer "F.Cu") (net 28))
 (via (at 132.858 79.0257) (size 0.8) (drill 0.4) (layers "F.Cu" "B.Cu") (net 28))
 (segment (start 146.8788 97.059) (end 146.8788 101.6254) (width 0.127) (layer "B.Cu") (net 28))
 (segment (start 132.858 83.0382) (end 146.8788 97.059) (width 0.127) (layer "B.Cu") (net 28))
 (segment (start 132.858 79.0257) (end 132.858 83.0382) (width 0.127) (layer "B.Cu") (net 28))
 (segment (start 147.8194 99.2004) (end 149.8038 99.2004) (width 0.127) (layer "F.Cu") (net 29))
 (segment (start 142.6789 94.0599) (end 147.8194 99.2004) (width 0.127) (layer "F.Cu") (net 29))
 (via (at 142.6789 94.0599) (size 0.8) (drill 0.4) (layers "F.Cu" "B.Cu") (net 29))
 (segment (start 130.8788 76.2754) (end 130.8788 82.2598) (width 0.127) (layer "B.Cu") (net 29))
 (segment (start 130.8788 82.2598) (end 142.6789 94.0599) (width 0.127) (layer "B.Cu") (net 29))
 (segment (start 133.2698 79.4395) (end 133.4418 79.2675) (width 0.127) (layer "B.Cu") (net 30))
 (segment (start 133.4418 79.2675) (end 133.4418 78.7722) (width 0.127) (layer "B.Cu") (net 30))
 (segment (start 133.2698 83.1002) (end 133.2698 79.4395) (width 0.127) (layer "B.Cu") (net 30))
 (segment (start 148.87 98.7004) (end 133.2698 83.1002) (width 0.127) (layer "B.Cu") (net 30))
 (segment (start 149.8038 98.7004) (end 148.87 98.7004) (width 0.127) (layer "B.Cu") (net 30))
 (segment (start 133.4418 78.7722) (end 131.8788 77.2092) (width 0.127) (layer "B.Cu") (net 30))
 (segment (start 131.8788 76.2754) (end 131.8788 77.2092) (width 0.127) (layer "B.Cu") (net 30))
 (segment (start 149.8038 98.2004) (end 148.87 98.2004) (width 0.127) (layer "F.Cu") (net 31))
 (segment (start 147.5127 96.8431) (end 147.5127 93.8829) (width 0.127) (layer "F.Cu") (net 31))
 (segment (start 148.87 98.2004) (end 147.5127 96.8431) (width 0.127) (layer "F.Cu") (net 31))
 (via (at 147.5127 93.8829) (size 0.8) (drill 0.4) (layers "F.Cu" "B.Cu") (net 31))
 (segment (start 137.8764 84.2466) (end 147.5127 93.8829) (width 0.127) (layer "B.Cu") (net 31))
 (segment (start 134.3788 76.2754) (end 134.3788 77.2092) (width 0.127) (layer "B.Cu") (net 31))
 (segment (start 134.3788 77.2092) (end 137.8764 80.7068) (width 0.127) (layer "B.Cu") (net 31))
 (segment (start 137.8764 80.7068) (end 137.8764 84.2466) (width 0.127) (layer "B.Cu") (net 31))
 (segment (start 130.3788 77.2092) (end 130.3788 77.372) (width 0.127) (layer "F.Cu") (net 32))
 (segment (start 130.3788 77.372) (end 133.2414 80.2346) (width 0.127) (layer "F.Cu") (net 32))
 (segment (start 130.3788 76.2754) (end 130.3788 77.2092) (width 0.127) (layer "F.Cu") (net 32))
 (segment (start 133.2414 80.2346) (end 133.8537 80.2346) (width 0.127) (layer "F.Cu") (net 32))
 (via (at 133.8537 80.2346) (size 0.8) (drill 0.4) (layers "F.Cu" "B.Cu") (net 32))
 (segment (start 148.87 97.7004) (end 133.8537 82.6841) (width 0.127) (layer "B.Cu") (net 32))
 (segment (start 149.8038 97.7004) (end 148.87 97.7004) (width 0.127) (layer "B.Cu") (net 32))
 (segment (start 133.8537 82.6841) (end 133.8537 80.2346) (width 0.127) (layer "B.Cu") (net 32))
 (segment (start 132.3788 76.2754) (end 132.3788 77.2092) (width 0.127) (layer "B.Cu") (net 33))
 (segment (start 134.4375 79.2679) (end 132.3788 77.2092) (width 0.127) (layer "B.Cu") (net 33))
 (segment (start 148.87 97.2004) (end 134.4375 82.7679) (width 0.127) (layer "B.Cu") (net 33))
 (segment (start 134.4375 82.7679) (end 134.4375 79.2679) (width 0.127) (layer "B.Cu") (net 33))
 (segment (start 149.8038 97.2004) (end 148.87 97.2004) (width 0.127) (layer "B.Cu") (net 33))
 (segment (start 148.87 96.7004) (end 148.1622 95.9926) (width 0.127) (layer "F.Cu") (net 34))
 (segment (start 149.8038 96.7004) (end 148.87 96.7004) (width 0.127) (layer "F.Cu") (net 34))
 (segment (start 148.1622 95.9926) (end 148.1622 94.9433) (width 0.127) (layer "F.Cu") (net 34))
 (via (at 148.1622 94.9433) (size 0.8) (drill 0.4) (layers "F.Cu" "B.Cu") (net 34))
 (segment (start 147.7417 94.9433) (end 135.1794 82.381) (width 0.127) (layer "B.Cu") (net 34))
 (segment (start 133.8788 76.2754) (end 133.8788 77.2092) (width 0.127) (layer "B.Cu") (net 34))
 (segment (start 148.1622 94.9433) (end 147.7417 94.9433) (width 0.127) (layer "B.Cu") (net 34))
 (segment (start 135.1794 78.5098) (end 133.8788 77.2092) (width 0.127) (layer "B.Cu") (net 34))
 (segment (start 135.1794 82.381) (end 135.1794 78.5098) (width 0.127) (layer "B.Cu") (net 34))
 (segment (start 148.87 94.3943) (end 148.87 96.2004) (width 0.127) (layer "F.Cu") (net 35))
 (segment (start 149.8038 96.2004) (end 148.87 96.2004) (width 0.127) (layer "F.Cu") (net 35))
 (segment (start 139.6102 93.1228) (end 147.5985 93.1228) (width 0.127) (layer "F.Cu") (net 35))
 (segment (start 147.5985 93.1228) (end 148.87 94.3943) (width 0.127) (layer "F.Cu") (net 35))
 (segment (start 136.3046 89.8172) (end 139.6102 93.1228) (width 0.127) (layer "F.Cu") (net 35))
 (via (at 136.3046 89.8172) (size 0.8) (drill 0.4) (layers "F.Cu" "B.Cu") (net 35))
 (segment (start 129.8788 83.3914) (end 136.3046 89.8172) (width 0.127) (layer "B.Cu") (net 35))
 (segment (start 129.8788 76.2754) (end 129.8788 83.3914) (width 0.127) (layer "B.Cu") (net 35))
 (segment (start 149.8038 95.7004) (end 148.87 95.7004) (width 0.127) (layer "B.Cu") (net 36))
 (segment (start 148.7789 95.7915) (end 147.811 95.7915) (width 0.127) (layer "B.Cu") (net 36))
 (segment (start 132.8788 76.2754) (end 132.8788 77.2092) (width 0.127) (layer "B.Cu") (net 36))
 (segment (start 134.6848 82.6653) (end 134.6848 79.0152) (width 0.127) (layer "B.Cu") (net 36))
 (segment (start 134.6848 79.0152) (end 132.8788 77.2092) (width 0.127) (layer "B.Cu") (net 36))
 (segment (start 148.87 95.7004) (end 148.7789 95.7915) (width 0.127) (layer "B.Cu") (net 36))
 (segment (start 147.811 95.7915) (end 134.6848 82.6653) (width 0.127) (layer "B.Cu") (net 36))
 (segment (start 134.9321 78.7625) (end 133.3788 77.2092) (width 0.127) (layer "B.Cu") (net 37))
 (segment (start 134.9321 82.5431) (end 134.9321 78.7625) (width 0.127) (layer "B.Cu") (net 37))
 (segment (start 148.87 95.2004) (end 148.5369 95.5335) (width 0.127) (layer "B.Cu") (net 37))
 (segment (start 149.8038 95.2004) (end 148.87 95.2004) (width 0.127) (layer "B.Cu") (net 37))
 (segment (start 133.3788 76.2754) (end 133.3788 77.2092) (width 0.127) (layer "B.Cu") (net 37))
 (segment (start 148.5369 95.5335) (end 147.9225 95.5335) (width 0.127) (layer "B.Cu") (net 37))
 (segment (start 147.9225 95.5335) (end 134.9321 82.5431) (width 0.127) (layer "B.Cu") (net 37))
 (segment (start 129.3788 77.2092) (end 136.2835 84.1139) (width 0.127) (layer "F.Cu") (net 38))
 (segment (start 136.2835 84.1139) (end 138.6612 84.1139) (width 0.127) (layer "F.Cu") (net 38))
 (segment (start 129.3788 76.2754) (end 129.3788 77.2092) (width 0.127) (layer "F.Cu") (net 38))
 (via (at 138.6612 84.1139) (size 0.8) (drill 0.4) (layers "F.Cu" "B.Cu") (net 38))
 (segment (start 149.8038 94.7004) (end 148.87 94.7004) (width 0.127) (layer "B.Cu") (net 38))
 (segment (start 148.87 94.3227) (end 148.87 94.7004) (width 0.127) (layer "B.Cu") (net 38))
 (segment (start 138.6612 84.1139) (end 148.87 94.3227) (width 0.127) (layer "B.Cu") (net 38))
 (segment (start 135.8788 78.2092) (end 148.87 91.2004) (width 0.127) (layer "B.Cu") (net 42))
 (segment (start 149.8038 91.2004) (end 148.87 91.2004) (width 0.127) (layer "B.Cu") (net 42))
 (segment (start 135.8788 76.2754) (end 135.8788 78.2092) (width 0.127) (layer "B.Cu") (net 42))
 (segment (start 137.3788 76.2754) (end 137.3788 78.3487) (width 0.127) (layer "F.Cu") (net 43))
 (segment (start 137.3788 78.3487) (end 141.1947 82.1646) (width 0.127) (layer "F.Cu") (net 43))
 (via (at 141.1947 82.1646) (size 0.8) (drill 0.4) (layers "F.Cu" "B.Cu") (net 43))
 (segment (start 149.8038 90.7004) (end 148.87 90.7004) (width 0.127) (layer "B.Cu") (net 43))
 (segment (start 141.1947 83.0251) (end 148.87 90.7004) (width 0.127) (layer "B.Cu") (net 43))
 (segment (start 141.1947 82.1646) (end 141.1947 83.0251) (width 0.127) (layer "B.Cu") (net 43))
 (segment (start 147.5909 87.7004) (end 141.0142 81.1237) (width 0.127) (layer "B.Cu") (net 47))
 (segment (start 149.8038 87.7004) (end 147.5909 87.7004) (width 0.127) (layer "B.Cu") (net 47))
 (segment (start 140.2933 81.1237) (end 136.3788 77.2092) (width 0.127) (layer "B.Cu") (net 47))
 (segment (start 136.3788 76.2754) (end 136.3788 77.2092) (width 0.127) (layer "B.Cu") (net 47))
 (segment (start 141.0142 81.1237) (end 140.2933 81.1237) (width 0.127) (layer "B.Cu") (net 47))
 (segment (start 127.3788 76.2754) (end 127.3788 77.2092) (width 0.127) (layer "F.Cu") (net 48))
 (segment (start 137.37 87.2004) (end 149.8038 87.2004) (width 0.127) (layer "F.Cu") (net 48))
 (segment (start 127.3788 77.2092) (end 137.37 87.2004) (width 0.127) (layer "F.Cu") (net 48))
 (segment (start 137.37 86.7004) (end 149.8038 86.7004) (width 0.127) (layer "F.Cu") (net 49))
 (segment (start 127.8788 76.2754) (end 127.8788 77.2092) (width 0.127) (layer "F.Cu") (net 49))
 (segment (start 127.8788 77.2092) (end 137.37 86.7004) (width 0.127) (layer "F.Cu") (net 49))
 (segment (start 128.3788 76.2754) (end 128.3788 77.2092) (width 0.127) (layer "F.Cu") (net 50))
 (segment (start 149.8038 86.2004) (end 137.37 86.2004) (width 0.127) (layer "F.Cu") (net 50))
 (segment (start 137.37 86.2004) (end 128.3788 77.2092) (width 0.127) (layer "F.Cu") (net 50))
 (segment (start 128.8788 77.2092) (end 137.37 85.7004) (width 0.127) (layer "F.Cu") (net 51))
 (segment (start 137.37 85.7004) (end 149.8038 85.7004) (width 0.127) (layer "F.Cu") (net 51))
 (segment (start 128.8788 76.2754) (end 128.8788 77.2092) (width 0.127) (layer "F.Cu") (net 51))
 (segment (start 136.8788 76.2754) (end 136.8788 77.2092) (width 0.127) (layer "B.Cu") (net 52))
 (segment (start 145.4406 85.2004) (end 137.4494 77.2092) (width 0.127) (layer "B.Cu") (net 52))
 (segment (start 149.8038 85.2004) (end 145.4406 85.2004) (width 0.127) (layer "B.Cu") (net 52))
 (segment (start 137.4494 77.2092) (end 136.8788 77.2092) (width 0.127) (layer "B.Cu") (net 52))
 (segment (start 149.8038 84.2004) (end 148.87 84.2004) (width 0.127) (layer "F.Cu") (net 54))
 (segment (start 142.37 84.2004) (end 148.87 84.2004) (width 0.127) (layer "F.Cu") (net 54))
 (segment (start 135.3788 76.2754) (end 135.3788 77.2092) (width 0.127) (layer "F.Cu") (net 54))
 (segment (start 135.3788 77.2092) (end 142.37 84.2004) (width 0.127) (layer "F.Cu") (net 54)))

